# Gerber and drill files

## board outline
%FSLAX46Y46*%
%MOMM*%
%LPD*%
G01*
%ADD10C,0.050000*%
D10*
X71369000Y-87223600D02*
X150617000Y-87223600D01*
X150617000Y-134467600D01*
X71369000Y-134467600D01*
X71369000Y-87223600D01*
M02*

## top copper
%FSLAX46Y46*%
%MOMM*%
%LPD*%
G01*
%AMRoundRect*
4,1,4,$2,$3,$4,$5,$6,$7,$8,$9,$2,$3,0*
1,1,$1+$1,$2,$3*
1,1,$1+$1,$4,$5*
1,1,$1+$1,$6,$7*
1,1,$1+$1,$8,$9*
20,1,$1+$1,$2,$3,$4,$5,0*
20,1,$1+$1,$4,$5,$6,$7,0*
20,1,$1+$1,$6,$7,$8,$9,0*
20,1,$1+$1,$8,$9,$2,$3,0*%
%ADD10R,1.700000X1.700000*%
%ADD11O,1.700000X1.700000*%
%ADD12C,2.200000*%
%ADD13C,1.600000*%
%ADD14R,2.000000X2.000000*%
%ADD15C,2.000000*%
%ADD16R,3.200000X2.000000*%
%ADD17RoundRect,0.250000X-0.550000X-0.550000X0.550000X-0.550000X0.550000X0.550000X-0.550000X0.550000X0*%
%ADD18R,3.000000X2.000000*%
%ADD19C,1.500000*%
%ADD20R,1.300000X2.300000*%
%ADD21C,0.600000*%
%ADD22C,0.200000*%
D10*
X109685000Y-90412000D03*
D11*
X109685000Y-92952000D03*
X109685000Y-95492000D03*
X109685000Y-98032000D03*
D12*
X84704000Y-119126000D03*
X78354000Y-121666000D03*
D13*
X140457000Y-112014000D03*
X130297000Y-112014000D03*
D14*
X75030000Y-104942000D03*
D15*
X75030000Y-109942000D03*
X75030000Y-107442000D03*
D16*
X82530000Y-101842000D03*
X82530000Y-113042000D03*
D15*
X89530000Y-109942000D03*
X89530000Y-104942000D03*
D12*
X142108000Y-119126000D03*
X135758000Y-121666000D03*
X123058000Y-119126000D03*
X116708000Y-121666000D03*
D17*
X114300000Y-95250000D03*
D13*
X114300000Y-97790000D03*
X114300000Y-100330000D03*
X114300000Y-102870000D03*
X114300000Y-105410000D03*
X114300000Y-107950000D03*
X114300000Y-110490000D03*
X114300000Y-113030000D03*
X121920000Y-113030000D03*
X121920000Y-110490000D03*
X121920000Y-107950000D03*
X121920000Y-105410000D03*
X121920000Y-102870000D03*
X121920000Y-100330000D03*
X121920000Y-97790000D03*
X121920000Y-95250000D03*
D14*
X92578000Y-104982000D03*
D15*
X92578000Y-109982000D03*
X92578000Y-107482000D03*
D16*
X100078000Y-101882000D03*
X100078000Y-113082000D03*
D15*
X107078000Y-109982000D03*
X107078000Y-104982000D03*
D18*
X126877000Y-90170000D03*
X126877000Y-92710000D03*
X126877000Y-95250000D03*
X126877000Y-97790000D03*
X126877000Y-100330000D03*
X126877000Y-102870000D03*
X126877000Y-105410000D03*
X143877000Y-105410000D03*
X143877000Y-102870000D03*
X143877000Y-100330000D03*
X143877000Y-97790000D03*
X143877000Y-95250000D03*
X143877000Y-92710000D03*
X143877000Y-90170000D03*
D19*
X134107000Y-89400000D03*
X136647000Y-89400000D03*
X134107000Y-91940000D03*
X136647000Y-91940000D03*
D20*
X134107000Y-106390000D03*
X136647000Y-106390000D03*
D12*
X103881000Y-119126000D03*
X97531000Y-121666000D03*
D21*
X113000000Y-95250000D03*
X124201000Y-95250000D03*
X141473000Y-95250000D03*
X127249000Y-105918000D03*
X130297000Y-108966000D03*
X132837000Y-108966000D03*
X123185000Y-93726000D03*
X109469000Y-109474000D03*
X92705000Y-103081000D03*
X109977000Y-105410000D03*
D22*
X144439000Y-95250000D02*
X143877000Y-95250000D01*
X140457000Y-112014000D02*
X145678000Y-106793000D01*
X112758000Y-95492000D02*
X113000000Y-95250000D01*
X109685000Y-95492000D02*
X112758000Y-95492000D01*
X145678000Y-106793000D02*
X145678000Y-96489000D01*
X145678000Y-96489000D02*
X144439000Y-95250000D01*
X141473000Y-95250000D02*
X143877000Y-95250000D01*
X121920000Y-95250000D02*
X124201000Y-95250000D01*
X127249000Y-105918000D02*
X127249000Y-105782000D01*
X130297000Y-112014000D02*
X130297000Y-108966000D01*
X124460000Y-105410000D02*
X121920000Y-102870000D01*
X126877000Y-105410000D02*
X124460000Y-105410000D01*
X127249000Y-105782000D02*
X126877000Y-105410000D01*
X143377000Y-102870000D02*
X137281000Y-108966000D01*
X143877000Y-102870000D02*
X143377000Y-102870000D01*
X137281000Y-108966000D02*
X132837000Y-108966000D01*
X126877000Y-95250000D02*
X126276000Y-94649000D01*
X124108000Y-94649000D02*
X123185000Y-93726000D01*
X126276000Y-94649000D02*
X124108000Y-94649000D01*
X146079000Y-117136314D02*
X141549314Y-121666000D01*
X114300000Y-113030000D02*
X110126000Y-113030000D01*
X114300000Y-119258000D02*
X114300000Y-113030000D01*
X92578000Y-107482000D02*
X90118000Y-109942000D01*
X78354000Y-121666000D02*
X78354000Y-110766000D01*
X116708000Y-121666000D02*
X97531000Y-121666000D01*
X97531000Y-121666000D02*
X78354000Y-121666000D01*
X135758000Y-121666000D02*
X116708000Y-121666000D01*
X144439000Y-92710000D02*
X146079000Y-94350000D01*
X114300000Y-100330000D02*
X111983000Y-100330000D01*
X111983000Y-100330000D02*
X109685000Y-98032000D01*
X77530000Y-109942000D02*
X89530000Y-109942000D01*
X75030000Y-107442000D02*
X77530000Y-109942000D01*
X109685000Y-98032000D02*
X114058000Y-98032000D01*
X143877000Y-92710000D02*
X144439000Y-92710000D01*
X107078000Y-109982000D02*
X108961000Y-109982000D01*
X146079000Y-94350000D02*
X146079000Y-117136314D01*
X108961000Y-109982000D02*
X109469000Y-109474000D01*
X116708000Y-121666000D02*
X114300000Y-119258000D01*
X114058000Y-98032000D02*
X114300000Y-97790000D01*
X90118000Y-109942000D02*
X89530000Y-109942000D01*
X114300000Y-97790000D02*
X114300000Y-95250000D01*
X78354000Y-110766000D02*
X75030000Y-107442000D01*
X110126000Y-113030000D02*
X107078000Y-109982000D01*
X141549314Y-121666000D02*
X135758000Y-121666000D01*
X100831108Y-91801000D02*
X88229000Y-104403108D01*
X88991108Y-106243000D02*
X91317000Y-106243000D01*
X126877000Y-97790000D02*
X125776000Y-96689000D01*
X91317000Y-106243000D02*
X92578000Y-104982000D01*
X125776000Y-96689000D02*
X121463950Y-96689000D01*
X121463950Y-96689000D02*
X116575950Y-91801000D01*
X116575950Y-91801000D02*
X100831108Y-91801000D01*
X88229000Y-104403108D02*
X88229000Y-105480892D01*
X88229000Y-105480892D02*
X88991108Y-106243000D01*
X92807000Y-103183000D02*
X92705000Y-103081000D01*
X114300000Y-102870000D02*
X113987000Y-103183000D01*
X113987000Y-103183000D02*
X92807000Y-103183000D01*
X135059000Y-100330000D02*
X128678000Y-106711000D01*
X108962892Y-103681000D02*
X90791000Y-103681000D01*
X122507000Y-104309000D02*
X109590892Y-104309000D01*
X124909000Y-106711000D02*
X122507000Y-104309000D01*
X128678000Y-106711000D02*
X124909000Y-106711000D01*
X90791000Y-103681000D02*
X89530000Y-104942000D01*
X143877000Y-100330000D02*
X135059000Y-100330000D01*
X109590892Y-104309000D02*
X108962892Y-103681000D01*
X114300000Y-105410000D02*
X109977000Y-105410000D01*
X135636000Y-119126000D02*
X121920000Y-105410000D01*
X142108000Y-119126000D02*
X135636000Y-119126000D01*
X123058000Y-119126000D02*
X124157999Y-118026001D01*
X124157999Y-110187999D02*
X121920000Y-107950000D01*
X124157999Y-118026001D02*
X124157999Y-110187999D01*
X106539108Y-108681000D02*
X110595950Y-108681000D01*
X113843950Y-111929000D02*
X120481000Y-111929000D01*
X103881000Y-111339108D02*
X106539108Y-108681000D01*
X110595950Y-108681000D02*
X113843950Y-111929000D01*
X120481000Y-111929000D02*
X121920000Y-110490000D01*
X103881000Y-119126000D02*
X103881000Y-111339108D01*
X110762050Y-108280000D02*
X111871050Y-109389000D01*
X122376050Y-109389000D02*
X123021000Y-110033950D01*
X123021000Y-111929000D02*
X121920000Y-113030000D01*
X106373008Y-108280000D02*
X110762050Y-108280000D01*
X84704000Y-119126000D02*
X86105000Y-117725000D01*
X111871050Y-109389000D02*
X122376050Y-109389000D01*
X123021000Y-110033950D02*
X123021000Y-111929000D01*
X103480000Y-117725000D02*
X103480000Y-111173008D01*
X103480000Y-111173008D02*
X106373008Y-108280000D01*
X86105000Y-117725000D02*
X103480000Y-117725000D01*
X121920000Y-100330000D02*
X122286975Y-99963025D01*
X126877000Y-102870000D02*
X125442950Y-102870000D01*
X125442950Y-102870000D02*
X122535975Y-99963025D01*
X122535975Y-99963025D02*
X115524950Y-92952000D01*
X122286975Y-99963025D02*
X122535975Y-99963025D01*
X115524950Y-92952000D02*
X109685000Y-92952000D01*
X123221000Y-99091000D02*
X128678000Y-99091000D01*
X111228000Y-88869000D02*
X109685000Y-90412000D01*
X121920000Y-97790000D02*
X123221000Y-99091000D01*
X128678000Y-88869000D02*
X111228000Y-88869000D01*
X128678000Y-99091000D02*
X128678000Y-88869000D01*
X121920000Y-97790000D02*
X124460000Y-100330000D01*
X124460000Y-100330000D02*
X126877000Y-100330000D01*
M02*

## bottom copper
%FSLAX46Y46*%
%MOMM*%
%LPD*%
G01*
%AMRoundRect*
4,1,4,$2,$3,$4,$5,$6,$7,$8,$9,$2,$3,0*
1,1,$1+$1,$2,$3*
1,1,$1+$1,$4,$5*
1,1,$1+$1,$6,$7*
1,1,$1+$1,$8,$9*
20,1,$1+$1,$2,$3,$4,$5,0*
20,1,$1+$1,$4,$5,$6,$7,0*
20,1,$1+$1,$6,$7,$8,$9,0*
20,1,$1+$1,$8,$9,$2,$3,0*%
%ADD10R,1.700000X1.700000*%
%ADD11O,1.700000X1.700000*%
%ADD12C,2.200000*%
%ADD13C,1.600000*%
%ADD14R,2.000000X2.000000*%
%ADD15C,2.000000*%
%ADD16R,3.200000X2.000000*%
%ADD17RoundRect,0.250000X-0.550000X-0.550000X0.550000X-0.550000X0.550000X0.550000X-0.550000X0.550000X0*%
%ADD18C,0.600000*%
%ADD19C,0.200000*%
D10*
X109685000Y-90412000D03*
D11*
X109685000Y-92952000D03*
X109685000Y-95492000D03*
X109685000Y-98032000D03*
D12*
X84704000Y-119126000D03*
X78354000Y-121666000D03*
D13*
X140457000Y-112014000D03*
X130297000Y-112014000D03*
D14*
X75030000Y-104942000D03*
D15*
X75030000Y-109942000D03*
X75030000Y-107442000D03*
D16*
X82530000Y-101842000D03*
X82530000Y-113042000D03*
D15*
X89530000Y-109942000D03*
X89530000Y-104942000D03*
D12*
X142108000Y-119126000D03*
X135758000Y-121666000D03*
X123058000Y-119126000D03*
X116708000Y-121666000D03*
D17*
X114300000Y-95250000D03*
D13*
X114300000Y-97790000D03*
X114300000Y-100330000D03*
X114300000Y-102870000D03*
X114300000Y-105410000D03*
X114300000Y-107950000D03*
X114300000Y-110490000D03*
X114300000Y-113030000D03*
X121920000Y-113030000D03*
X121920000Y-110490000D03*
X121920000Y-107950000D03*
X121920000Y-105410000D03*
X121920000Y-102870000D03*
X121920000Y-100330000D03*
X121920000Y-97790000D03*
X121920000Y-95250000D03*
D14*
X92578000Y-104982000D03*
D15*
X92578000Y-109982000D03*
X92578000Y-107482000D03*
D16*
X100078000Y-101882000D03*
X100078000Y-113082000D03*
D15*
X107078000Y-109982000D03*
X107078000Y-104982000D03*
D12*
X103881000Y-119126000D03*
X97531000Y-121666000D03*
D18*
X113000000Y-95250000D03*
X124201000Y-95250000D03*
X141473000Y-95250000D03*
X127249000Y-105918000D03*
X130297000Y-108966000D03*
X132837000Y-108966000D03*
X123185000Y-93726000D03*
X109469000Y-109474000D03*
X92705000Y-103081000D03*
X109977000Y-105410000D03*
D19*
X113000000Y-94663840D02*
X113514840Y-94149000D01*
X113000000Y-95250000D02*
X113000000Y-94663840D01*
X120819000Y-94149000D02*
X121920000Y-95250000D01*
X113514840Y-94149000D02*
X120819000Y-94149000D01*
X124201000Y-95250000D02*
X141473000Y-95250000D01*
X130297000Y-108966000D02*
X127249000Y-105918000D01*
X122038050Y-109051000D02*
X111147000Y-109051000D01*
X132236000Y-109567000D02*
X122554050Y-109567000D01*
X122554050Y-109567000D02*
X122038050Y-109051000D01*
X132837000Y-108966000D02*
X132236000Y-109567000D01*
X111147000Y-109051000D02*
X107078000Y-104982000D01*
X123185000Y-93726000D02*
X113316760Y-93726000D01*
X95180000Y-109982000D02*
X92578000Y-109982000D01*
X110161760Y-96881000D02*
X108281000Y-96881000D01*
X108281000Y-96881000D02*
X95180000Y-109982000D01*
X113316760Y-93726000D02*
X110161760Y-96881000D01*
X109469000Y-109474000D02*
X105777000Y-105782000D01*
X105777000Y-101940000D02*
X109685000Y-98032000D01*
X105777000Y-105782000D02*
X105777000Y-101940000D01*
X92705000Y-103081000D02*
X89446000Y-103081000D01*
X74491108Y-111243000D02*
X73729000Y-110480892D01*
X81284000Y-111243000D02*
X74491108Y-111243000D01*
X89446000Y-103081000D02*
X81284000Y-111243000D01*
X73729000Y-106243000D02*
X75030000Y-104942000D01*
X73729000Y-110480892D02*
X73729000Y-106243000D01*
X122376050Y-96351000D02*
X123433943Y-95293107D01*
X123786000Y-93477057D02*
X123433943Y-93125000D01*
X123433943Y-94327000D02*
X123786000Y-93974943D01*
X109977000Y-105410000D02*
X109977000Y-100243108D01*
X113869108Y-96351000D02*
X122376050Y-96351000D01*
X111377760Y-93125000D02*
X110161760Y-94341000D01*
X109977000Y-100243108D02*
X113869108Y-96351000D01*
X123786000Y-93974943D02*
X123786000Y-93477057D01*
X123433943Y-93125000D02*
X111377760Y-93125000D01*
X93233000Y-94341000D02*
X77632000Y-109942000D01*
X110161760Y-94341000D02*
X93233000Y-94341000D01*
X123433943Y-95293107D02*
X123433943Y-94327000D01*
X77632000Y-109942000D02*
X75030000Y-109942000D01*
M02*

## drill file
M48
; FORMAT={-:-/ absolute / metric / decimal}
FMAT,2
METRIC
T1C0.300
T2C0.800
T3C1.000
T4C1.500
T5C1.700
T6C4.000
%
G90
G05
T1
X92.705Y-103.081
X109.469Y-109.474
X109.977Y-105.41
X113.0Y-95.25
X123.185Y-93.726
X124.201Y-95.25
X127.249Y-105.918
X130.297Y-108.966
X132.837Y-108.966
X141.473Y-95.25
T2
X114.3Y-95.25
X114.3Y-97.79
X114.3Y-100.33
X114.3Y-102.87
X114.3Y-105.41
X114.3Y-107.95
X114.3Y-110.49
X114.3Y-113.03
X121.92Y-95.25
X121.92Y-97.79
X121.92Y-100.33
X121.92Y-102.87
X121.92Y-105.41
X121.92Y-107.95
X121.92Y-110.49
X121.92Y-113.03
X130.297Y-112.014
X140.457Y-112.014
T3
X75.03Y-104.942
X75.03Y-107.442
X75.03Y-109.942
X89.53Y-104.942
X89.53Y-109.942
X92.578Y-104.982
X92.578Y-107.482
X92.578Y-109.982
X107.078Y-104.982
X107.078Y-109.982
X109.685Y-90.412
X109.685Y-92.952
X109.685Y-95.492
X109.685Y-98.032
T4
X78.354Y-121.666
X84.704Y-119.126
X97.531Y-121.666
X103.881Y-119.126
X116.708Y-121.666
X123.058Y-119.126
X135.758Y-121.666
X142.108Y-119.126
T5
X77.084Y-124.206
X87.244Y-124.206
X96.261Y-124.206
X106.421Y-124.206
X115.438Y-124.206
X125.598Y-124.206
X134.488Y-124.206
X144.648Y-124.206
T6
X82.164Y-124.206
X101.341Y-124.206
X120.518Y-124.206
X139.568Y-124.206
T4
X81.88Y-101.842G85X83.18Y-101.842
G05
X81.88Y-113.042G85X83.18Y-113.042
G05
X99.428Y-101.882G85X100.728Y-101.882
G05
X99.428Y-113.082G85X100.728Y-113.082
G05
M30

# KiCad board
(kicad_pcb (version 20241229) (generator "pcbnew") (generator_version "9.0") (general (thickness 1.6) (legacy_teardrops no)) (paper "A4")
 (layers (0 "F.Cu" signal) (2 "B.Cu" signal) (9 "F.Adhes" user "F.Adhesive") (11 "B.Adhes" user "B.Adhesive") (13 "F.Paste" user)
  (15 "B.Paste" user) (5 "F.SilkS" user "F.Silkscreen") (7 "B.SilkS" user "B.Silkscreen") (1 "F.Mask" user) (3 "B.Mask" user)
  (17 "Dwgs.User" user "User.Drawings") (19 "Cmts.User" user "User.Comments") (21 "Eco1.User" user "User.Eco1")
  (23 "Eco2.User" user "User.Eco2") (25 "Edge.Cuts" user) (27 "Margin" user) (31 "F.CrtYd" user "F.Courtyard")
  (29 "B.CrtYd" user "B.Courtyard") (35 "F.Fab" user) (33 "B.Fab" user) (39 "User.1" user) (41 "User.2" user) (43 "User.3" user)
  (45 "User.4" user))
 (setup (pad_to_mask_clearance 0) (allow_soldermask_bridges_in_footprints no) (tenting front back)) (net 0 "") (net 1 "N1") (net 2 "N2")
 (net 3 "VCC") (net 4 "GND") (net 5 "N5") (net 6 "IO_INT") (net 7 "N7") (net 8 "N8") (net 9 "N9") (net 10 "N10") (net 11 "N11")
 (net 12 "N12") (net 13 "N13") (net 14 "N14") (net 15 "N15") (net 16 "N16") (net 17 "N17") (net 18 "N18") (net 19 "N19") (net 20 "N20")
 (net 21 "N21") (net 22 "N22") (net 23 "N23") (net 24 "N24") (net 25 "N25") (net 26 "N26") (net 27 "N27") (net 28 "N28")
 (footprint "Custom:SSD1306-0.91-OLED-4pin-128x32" (layer "F.Cu") (at 73.185 88.222)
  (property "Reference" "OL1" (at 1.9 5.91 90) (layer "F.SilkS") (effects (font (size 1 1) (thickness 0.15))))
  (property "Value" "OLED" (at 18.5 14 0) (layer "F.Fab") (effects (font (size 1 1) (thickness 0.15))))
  (pad "1" thru_hole rect (at 36.5 2.19) (size 1.7 1.7) (drill 1) (layers "*.Cu" "*.Mask") (remove_unused_layers no) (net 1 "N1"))
  (pad "2" thru_hole oval (at 36.5 4.73) (size 1.7 1.7) (drill 1) (layers "*.Cu" "*.Mask") (remove_unused_layers no) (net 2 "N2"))
  (pad "3" thru_hole oval (at 36.5 7.27) (size 1.7 1.7) (drill 1) (layers "*.Cu" "*.Mask") (remove_unused_layers no) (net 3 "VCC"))
  (pad "4" thru_hole oval (at 36.5 9.81) (size 1.7 1.7) (drill 1) (layers "*.Cu" "*.Mask") (remove_unused_layers no) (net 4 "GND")))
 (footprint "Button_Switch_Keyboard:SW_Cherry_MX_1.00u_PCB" (layer "F.Cu") (at 84.704 119.126)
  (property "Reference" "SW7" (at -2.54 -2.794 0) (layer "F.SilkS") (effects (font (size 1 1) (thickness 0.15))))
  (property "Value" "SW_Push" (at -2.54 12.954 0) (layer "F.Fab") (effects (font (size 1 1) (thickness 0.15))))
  (pad "" np_thru_hole circle (at -7.62 5.08) (size 1.7 1.7) (drill 1.7) (layers "*.Cu" "*.Mask"))
  (pad "" np_thru_hole circle (at -2.54 5.08) (size 4 4) (drill 4) (layers "*.Cu" "*.Mask"))
  (pad "" np_thru_hole circle (at 2.54 5.08) (size 1.7 1.7) (drill 1.7) (layers "*.Cu" "*.Mask"))
  (pad "1" thru_hole circle (at 0 0) (size 2.2 2.2) (drill 1.5) (layers "*.Cu" "*.Mask") (remove_unused_layers no) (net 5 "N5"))
  (pad "2" thru_hole circle (at -6.35 2.54) (size 2.2 2.2) (drill 1.5) (layers "*.Cu" "*.Mask") (remove_unused_layers no) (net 4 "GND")))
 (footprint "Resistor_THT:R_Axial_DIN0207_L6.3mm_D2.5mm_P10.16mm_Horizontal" (layer "F.Cu") (at 140.457 112.014 180)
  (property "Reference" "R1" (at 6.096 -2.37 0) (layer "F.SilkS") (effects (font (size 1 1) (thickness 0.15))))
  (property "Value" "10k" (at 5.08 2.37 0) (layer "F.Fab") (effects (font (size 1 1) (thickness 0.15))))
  (pad "1" thru_hole circle (at 0 0 180) (size 1.6 1.6) (drill 0.8) (layers "*.Cu" "*.Mask") (remove_unused_layers no) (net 3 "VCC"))
  (pad "2" thru_hole circle (at 10.16 0 180) (size 1.6 1.6) (drill 0.8) (layers "*.Cu" "*.Mask") (remove_unused_layers no) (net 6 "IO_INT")))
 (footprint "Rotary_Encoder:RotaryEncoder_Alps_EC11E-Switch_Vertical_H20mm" (layer "F.Cu") (at 75.03 104.942)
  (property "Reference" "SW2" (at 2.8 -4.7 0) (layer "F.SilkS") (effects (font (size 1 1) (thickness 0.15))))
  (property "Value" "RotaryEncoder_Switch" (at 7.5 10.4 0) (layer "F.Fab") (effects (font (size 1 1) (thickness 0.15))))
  (pad "A" thru_hole rect (at 0 0) (size 2 2) (drill 1) (layers "*.Cu" "*.Mask") (remove_unused_layers no) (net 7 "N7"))
  (pad "B" thru_hole circle (at 0 5) (size 2 2) (drill 1) (layers "*.Cu" "*.Mask") (remove_unused_layers no) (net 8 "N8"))
  (pad "C" thru_hole circle (at 0 2.5) (size 2 2) (drill 1) (layers "*.Cu" "*.Mask") (remove_unused_layers no) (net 4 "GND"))
  (pad "MP" thru_hole rect (at 7.5 -3.1) (size 3.2 2) (drill oval 2.8 1.5) (layers "*.Cu" "*.Mask") (remove_unused_layers no))
  (pad "MP" thru_hole rect (at 7.5 8.1) (size 3.2 2) (drill oval 2.8 1.5) (layers "*.Cu" "*.Mask") (remove_unused_layers no))
  (pad "S1" thru_hole circle (at 14.5 5) (size 2 2) (drill 1) (layers "*.Cu" "*.Mask") (remove_unused_layers no) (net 4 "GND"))
  (pad "S2" thru_hole circle (at 14.5 0) (size 2 2) (drill 1) (layers "*.Cu" "*.Mask") (remove_unused_layers no) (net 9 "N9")))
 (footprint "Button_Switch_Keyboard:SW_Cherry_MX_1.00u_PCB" (layer "F.Cu") (at 142.108 119.126)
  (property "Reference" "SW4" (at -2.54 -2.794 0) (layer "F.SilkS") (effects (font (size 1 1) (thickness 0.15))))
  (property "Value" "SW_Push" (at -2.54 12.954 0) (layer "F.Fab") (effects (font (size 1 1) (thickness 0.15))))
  (pad "" np_thru_hole circle (at -7.62 5.08) (size 1.7 1.7) (drill 1.7) (layers "*.Cu" "*.Mask"))
  (pad "" np_thru_hole circle (at -2.54 5.08) (size 4 4) (drill 4) (layers "*.Cu" "*.Mask"))
  (pad "" np_thru_hole circle (at 2.54 5.08) (size 1.7 1.7) (drill 1.7) (layers "*.Cu" "*.Mask"))
  (pad "1" thru_hole circle (at 0 0) (size 2.2 2.2) (drill 1.5) (layers "*.Cu" "*.Mask") (remove_unused_layers no) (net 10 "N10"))
  (pad "2" thru_hole circle (at -6.35 2.54) (size 2.2 2.2) (drill 1.5) (layers "*.Cu" "*.Mask") (remove_unused_layers no) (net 4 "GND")))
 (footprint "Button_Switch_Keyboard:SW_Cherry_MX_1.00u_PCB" (layer "F.Cu") (at 123.058 119.126)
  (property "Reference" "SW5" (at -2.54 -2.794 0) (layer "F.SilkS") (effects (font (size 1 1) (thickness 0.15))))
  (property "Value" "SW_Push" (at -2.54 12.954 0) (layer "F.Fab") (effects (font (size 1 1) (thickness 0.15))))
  (pad "" np_thru_hole circle (at -7.62 5.08) (size 1.7 1.7) (drill 1.7) (layers "*.Cu" "*.Mask"))
  (pad "" np_thru_hole circle (at -2.54 5.08) (size 4 4) (drill 4) (layers "*.Cu" "*.Mask"))
  (pad "" np_thru_hole circle (at 2.54 5.08) (size 1.7 1.7) (drill 1.7) (layers "*.Cu" "*.Mask"))
  (pad "1" thru_hole circle (at 0 0) (size 2.2 2.2) (drill 1.5) (layers "*.Cu" "*.Mask") (remove_unused_layers no) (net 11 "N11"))
  (pad "2" thru_hole circle (at -6.35 2.54) (size 2.2 2.2) (drill 1.5) (layers "*.Cu" "*.Mask") (remove_unused_layers no) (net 4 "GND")))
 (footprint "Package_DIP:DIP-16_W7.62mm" (layer "F.Cu") (at 114.3 95.25)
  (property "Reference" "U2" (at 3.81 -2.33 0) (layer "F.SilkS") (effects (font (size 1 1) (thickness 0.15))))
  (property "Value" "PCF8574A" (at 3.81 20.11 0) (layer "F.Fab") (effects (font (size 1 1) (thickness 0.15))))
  (pad "1" thru_hole roundrect (at 0 0) (size 1.6 1.6) (drill 0.8) (layers "*.Cu" "*.Mask") (remove_unused_layers no)
   (roundrect_rratio 0.15625) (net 4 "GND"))
  (pad "2" thru_hole circle (at 0 2.54) (size 1.6 1.6) (drill 0.8) (layers "*.Cu" "*.Mask") (remove_unused_layers no) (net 4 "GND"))
  (pad "3" thru_hole circle (at 0 5.08) (size 1.6 1.6) (drill 0.8) (layers "*.Cu" "*.Mask") (remove_unused_layers no) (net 4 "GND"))
  (pad "4" thru_hole circle (at 0 7.62) (size 1.6 1.6) (drill 0.8) (layers "*.Cu" "*.Mask") (remove_unused_layers no) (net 7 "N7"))
  (pad "5" thru_hole circle (at 0 10.16) (size 1.6 1.6) (drill 0.8) (layers "*.Cu" "*.Mask") (remove_unused_layers no) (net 8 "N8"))
  (pad "6" thru_hole circle (at 0 12.7) (size 1.6 1.6) (drill 0.8) (layers "*.Cu" "*.Mask") (remove_unused_layers no) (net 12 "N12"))
  (pad "7" thru_hole circle (at 0 15.24) (size 1.6 1.6) (drill 0.8) (layers "*.Cu" "*.Mask") (remove_unused_layers no) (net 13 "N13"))
  (pad "8" thru_hole circle (at 0 17.78) (size 1.6 1.6) (drill 0.8) (layers "*.Cu" "*.Mask") (remove_unused_layers no) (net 4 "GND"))
  (pad "9" thru_hole circle (at 7.62 17.78) (size 1.6 1.6) (drill 0.8) (layers "*.Cu" "*.Mask") (remove_unused_layers no) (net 5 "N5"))
  (pad "10" thru_hole circle (at 7.62 15.24) (size 1.6 1.6) (drill 0.8) (layers "*.Cu" "*.Mask") (remove_unused_layers no) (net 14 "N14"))
  (pad "11" thru_hole circle (at 7.62 12.7) (size 1.6 1.6) (drill 0.8) (layers "*.Cu" "*.Mask") (remove_unused_layers no) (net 11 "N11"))
  (pad "12" thru_hole circle (at 7.62 10.16) (size 1.6 1.6) (drill 0.8) (layers "*.Cu" "*.Mask") (remove_unused_layers no) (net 10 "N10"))
  (pad "13" thru_hole circle (at 7.62 7.62) (size 1.6 1.6) (drill 0.8) (layers "*.Cu" "*.Mask") (remove_unused_layers no) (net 6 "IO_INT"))
  (pad "14" thru_hole circle (at 7.62 5.08) (size 1.6 1.6) (drill 0.8) (layers "*.Cu" "*.Mask") (remove_unused_layers no) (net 2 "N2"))
  (pad "15" thru_hole circle (at 7.62 2.54) (size 1.6 1.6) (drill 0.8) (layers "*.Cu" "*.Mask") (remove_unused_layers no) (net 1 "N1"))
  (pad "16" thru_hole circle (at 7.62 0) (size 1.6 1.6) (drill 0.8) (layers "*.Cu" "*.Mask") (remove_unused_layers no) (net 3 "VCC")))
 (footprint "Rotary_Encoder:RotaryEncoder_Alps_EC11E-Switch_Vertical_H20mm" (layer "F.Cu") (at 92.578 104.982)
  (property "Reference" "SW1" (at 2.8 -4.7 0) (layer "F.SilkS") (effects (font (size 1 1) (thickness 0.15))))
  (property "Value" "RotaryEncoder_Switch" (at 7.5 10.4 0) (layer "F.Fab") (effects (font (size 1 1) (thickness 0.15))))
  (pad "A" thru_hole rect (at 0 0) (size 2 2) (drill 1) (layers "*.Cu" "*.Mask") (remove_unused_layers no) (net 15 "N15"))
  (pad "B" thru_hole circle (at 0 5) (size 2 2) (drill 1) (layers "*.Cu" "*.Mask") (remove_unused_layers no) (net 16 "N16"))
  (pad "C" thru_hole circle (at 0 2.5) (size 2 2) (drill 1) (layers "*.Cu" "*.Mask") (remove_unused_layers no) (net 4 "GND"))
  (pad "MP" thru_hole rect (at 7.5 -3.1) (size 3.2 2) (drill oval 2.8 1.5) (layers "*.Cu" "*.Mask") (remove_unused_layers no))
  (pad "MP" thru_hole rect (at 7.5 8.1) (size 3.2 2) (drill oval 2.8 1.5) (layers "*.Cu" "*.Mask") (remove_unused_layers no))
  (pad "S1" thru_hole circle (at 14.5 5) (size 2 2) (drill 1) (layers "*.Cu" "*.Mask") (remove_unused_layers no) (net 4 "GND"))
  (pad "S2" thru_hole circle (at 14.5 0) (size 2 2) (drill 1) (layers "*.Cu" "*.Mask") (remove_unused_layers no) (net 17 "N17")))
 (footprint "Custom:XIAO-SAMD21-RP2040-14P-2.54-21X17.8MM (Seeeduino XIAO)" (layer "F.Cu") (at 135.377 97.79)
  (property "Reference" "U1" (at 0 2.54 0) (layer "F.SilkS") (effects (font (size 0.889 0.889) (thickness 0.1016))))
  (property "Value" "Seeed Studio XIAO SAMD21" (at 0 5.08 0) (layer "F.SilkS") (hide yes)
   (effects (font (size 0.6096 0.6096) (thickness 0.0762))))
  (pad "1" smd rect (at -8.5 -7.62) (size 3 2) (layers "F.Cu" "F.Mask" "F.Paste") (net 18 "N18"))
  (pad "2" smd rect (at -8.5 -5.08) (size 3 2) (layers "F.Cu" "F.Mask" "F.Paste") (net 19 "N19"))
  (pad "3" smd rect (at -8.5 -2.54) (size 3 2) (layers "F.Cu" "F.Mask" "F.Paste") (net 16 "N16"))
  (pad "4" smd rect (at -8.5 0) (size 3 2) (layers "F.Cu" "F.Mask" "F.Paste") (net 15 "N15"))
  (pad "5" smd rect (at -8.5 2.54) (size 3 2) (layers "F.Cu" "F.Mask" "F.Paste") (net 1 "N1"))
  (pad "6" smd rect (at -8.5 5.08 180) (size 3 2) (layers "F.Cu" "F.Mask" "F.Paste") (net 2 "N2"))
  (pad "7" smd rect (at -8.5 7.62) (size 3 2) (layers "F.Cu" "F.Mask" "F.Paste") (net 6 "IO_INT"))
  (pad "8" smd rect (at 8.5 7.62) (size 3 2) (layers "F.Cu" "F.Mask" "F.Paste") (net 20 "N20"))
  (pad "9" smd rect (at 8.5 5.08) (size 3 2) (layers "F.Cu" "F.Mask" "F.Paste") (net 17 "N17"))
  (pad "10" smd rect (at 8.5 2.54) (size 3 2) (layers "F.Cu" "F.Mask" "F.Paste") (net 9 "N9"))
  (pad "11" smd rect (at 8.5 0) (size 3 2) (layers "F.Cu" "F.Mask" "F.Paste") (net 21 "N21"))
  (pad "12" smd rect (at 8.5 -2.54) (size 3 2) (layers "F.Cu" "F.Mask" "F.Paste") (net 3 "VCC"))
  (pad "13" smd rect (at 8.5 -5.08) (size 3 2) (layers "F.Cu" "F.Mask" "F.Paste") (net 4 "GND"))
  (pad "14" smd rect (at 8.5 -7.62) (size 3 2) (layers "F.Cu" "F.Mask" "F.Paste") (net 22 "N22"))
  (pad "15" smd circle (at -1.27 -8.39 90) (size 1.5 1.5) (layers "F.Cu" "F.Mask" "F.Paste") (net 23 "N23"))
  (pad "16" smd circle (at 1.27 -8.39 90) (size 1.5 1.5) (layers "F.Cu" "F.Mask" "F.Paste") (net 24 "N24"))
  (pad "17" smd circle (at -1.27 -5.85 90) (size 1.5 1.5) (layers "F.Cu" "F.Mask" "F.Paste") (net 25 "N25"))
  (pad "18" smd circle (at 1.27 -5.85 90) (size 1.5 1.5) (layers "F.Cu" "F.Mask" "F.Paste") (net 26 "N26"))
  (pad "19" smd rect (at -1.27 8.6 90) (size 2.3 1.3) (layers "F.Cu" "F.Mask" "F.Paste") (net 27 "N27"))
  (pad "20" smd rect (at 1.27 8.6 90) (size 2.3 1.3) (layers "F.Cu" "F.Mask" "F.Paste") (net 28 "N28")))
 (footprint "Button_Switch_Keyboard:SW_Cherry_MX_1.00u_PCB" (layer "F.Cu") (at 103.881 119.126)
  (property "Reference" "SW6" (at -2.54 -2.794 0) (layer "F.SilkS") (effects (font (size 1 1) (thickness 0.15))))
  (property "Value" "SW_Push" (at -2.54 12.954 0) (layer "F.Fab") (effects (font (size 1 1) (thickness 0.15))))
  (pad "" np_thru_hole circle (at -7.62 5.08) (size 1.7 1.7) (drill 1.7) (layers "*.Cu" "*.Mask"))
  (pad "" np_thru_hole circle (at -2.54 5.08) (size 4 4) (drill 4) (layers "*.Cu" "*.Mask"))
  (pad "" np_thru_hole circle (at 2.54 5.08) (size 1.7 1.7) (drill 1.7) (layers "*.Cu" "*.Mask"))
  (pad "1" thru_hole circle (at 0 0) (size 2.2 2.2) (drill 1.5) (layers "*.Cu" "*.Mask") (remove_unused_layers no) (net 14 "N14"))
  (pad "2" thru_hole circle (at -6.35 2.54) (size 2.2 2.2) (drill 1.5) (layers "*.Cu" "*.Mask") (remove_unused_layers no) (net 4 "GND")))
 (gr_rect (start 71.369 87.2236) (end 150.617 134.4676) (stroke (width 0.05) (type default)) (fill no) (layer "Edge.Cuts"))
 (segment (start 144.439 95.25) (end 143.877 95.25) (width 0.2) (layer "F.Cu") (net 3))
 (segment (start 140.457 112.014) (end 145.678 106.793) (width 0.2) (layer "F.Cu") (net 3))
 (segment (start 112.758 95.492) (end 113 95.25) (width 0.2) (layer "F.Cu") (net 3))
 (segment (start 109.685 95.492) (end 112.758 95.492) (width 0.2) (layer "F.Cu") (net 3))
 (segment (start 145.678 106.793) (end 145.678 96.489) (width 0.2) (layer "F.Cu") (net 3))
 (segment (start 145.678 96.489) (end 144.439 95.25) (width 0.2) (layer "F.Cu") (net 3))
 (segment (start 141.473 95.25) (end 143.877 95.25) (width 0.2) (layer "F.Cu") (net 3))
 (segment (start 121.92 95.25) (end 124.201 95.25) (width 0.2) (layer "F.Cu") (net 3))
 (via (at 113 95.25) (size 0.6) (drill 0.3) (layers "F.Cu" "B.Cu") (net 3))
 (via (at 124.201 95.25) (size 0.6) (drill 0.3) (layers "F.Cu" "B.Cu") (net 3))
 (via (at 141.473 95.25) (size 0.6) (drill 0.3) (layers "F.Cu" "B.Cu") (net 3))
 (segment (start 113 94.66384) (end 113.51484 94.149) (width 0.2) (layer "B.Cu") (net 3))
 (segment (start 113 95.25) (end 113 94.66384) (width 0.2) (layer "B.Cu") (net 3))
 (segment (start 120.819 94.149) (end 121.92 95.25) (width 0.2) (layer "B.Cu") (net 3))
 (segment (start 113.51484 94.149) (end 120.819 94.149) (width 0.2) (layer "B.Cu") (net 3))
 (segment (start 124.201 95.25) (end 141.473 95.25) (width 0.2) (layer "B.Cu") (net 3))
 (segment (start 127.249 105.918) (end 127.249 105.782) (width 0.2) (layer "F.Cu") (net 6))
 (segment (start 130.297 112.014) (end 130.297 108.966) (width 0.2) (layer "F.Cu") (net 6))
 (segment (start 124.46 105.41) (end 121.92 102.87) (width 0.2) (layer "F.Cu") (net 6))
 (segment (start 126.877 105.41) (end 124.46 105.41) (width 0.2) (layer "F.Cu") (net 6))
 (segment (start 127.249 105.782) (end 126.877 105.41) (width 0.2) (layer "F.Cu") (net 6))
 (via (at 127.249 105.918) (size 0.6) (drill 0.3) (layers "F.Cu" "B.Cu") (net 6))
 (via (at 130.297 108.966) (size 0.6) (drill 0.3) (layers "F.Cu" "B.Cu") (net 6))
 (segment (start 130.297 108.966) (end 127.249 105.918) (width 0.2) (layer "B.Cu") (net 6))
 (segment (start 143.377 102.87) (end 137.281 108.966) (width 0.2) (layer "F.Cu") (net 17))
 (segment (start 143.877 102.87) (end 143.377 102.87) (width 0.2) (layer "F.Cu") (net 17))
 (segment (start 137.281 108.966) (end 132.837 108.966) (width 0.2) (layer "F.Cu") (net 17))
 (via (at 132.837 108.966) (size 0.6) (drill 0.3) (layers "F.Cu" "B.Cu") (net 17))
 (segment (start 122.03805 109.051) (end 111.147 109.051) (width 0.2) (layer "B.Cu") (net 17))
 (segment (start 132.236 109.567) (end 122.55405 109.567) (width 0.2) (layer "B.Cu") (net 17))
 (segment (start 122.55405 109.567) (end 122.03805 109.051) (width 0.2) (layer "B.Cu") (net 17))
 (segment (start 132.837 108.966) (end 132.236 109.567) (width 0.2) (layer "B.Cu") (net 17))
 (segment (start 111.147 109.051) (end 107.078 104.982) (width 0.2) (layer "B.Cu") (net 17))
 (segment (start 126.877 95.25) (end 126.276 94.649) (width 0.2) (layer "F.Cu") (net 16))
 (segment (start 124.108 94.649) (end 123.185 93.726) (width 0.2) (layer "F.Cu") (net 16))
 (segment (start 126.276 94.649) (end 124.108 94.649) (width 0.2) (layer "F.Cu") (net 16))
 (via (at 123.185 93.726) (size 0.6) (drill 0.3) (layers "F.Cu" "B.Cu") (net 16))
 (segment (start 123.185 93.726) (end 113.31676 93.726) (width 0.2) (layer "B.Cu") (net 16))
 (segment (start 95.18 109.982) (end 92.578 109.982) (width 0.2) (layer "B.Cu") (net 16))
 (segment (start 110.16176 96.881) (end 108.281 96.881) (width 0.2) (layer "B.Cu") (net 16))
 (segment (start 108.281 96.881) (end 95.18 109.982) (width 0.2) (layer "B.Cu") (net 16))
 (segment (start 113.31676 93.726) (end 110.16176 96.881) (width 0.2) (layer "B.Cu") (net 16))
 (segment (start 146.079 117.136314) (end 141.549314 121.666) (width 0.2) (layer "F.Cu") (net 4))
 (segment (start 114.3 113.03) (end 110.126 113.03) (width 0.2) (layer "F.Cu") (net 4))
 (segment (start 114.3 119.258) (end 114.3 113.03) (width 0.2) (layer "F.Cu") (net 4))
 (segment (start 92.578 107.482) (end 90.118 109.942) (width 0.2) (layer "F.Cu") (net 4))
 (segment (start 78.354 121.666) (end 78.354 110.766) (width 0.2) (layer "F.Cu") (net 4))
 (segment (start 116.708 121.666) (end 97.531 121.666) (width 0.2) (layer "F.Cu") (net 4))
 (segment (start 97.531 121.666) (end 78.354 121.666) (width 0.2) (layer "F.Cu") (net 4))
 (segment (start 135.758 121.666) (end 116.708 121.666) (width 0.2) (layer "F.Cu") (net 4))
 (segment (start 144.439 92.71) (end 146.079 94.35) (width 0.2) (layer "F.Cu") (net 4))
 (segment (start 114.3 100.33) (end 111.983 100.33) (width 0.2) (layer "F.Cu") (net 4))
 (segment (start 111.983 100.33) (end 109.685 98.032) (width 0.2) (layer "F.Cu") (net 4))
 (segment (start 77.53 109.942) (end 89.53 109.942) (width 0.2) (layer "F.Cu") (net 4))
 (segment (start 75.03 107.442) (end 77.53 109.942) (width 0.2) (layer "F.Cu") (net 4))
 (segment (start 109.685 98.032) (end 114.058 98.032) (width 0.2) (layer "F.Cu") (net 4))
 (segment (start 143.877 92.71) (end 144.439 92.71) (width 0.2) (layer "F.Cu") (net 4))
 (segment (start 107.078 109.982) (end 108.961 109.982) (width 0.2) (layer "F.Cu") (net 4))
 (segment (start 146.079 94.35) (end 146.079 117.136314) (width 0.2) (layer "F.Cu") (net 4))
 (segment (start 108.961 109.982) (end 109.469 109.474) (width 0.2) (layer "F.Cu") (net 4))
 (segment (start 116.708 121.666) (end 114.3 119.258) (width 0.2) (layer "F.Cu") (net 4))
 (segment (start 114.058 98.032) (end 114.3 97.79) (width 0.2) (layer "F.Cu") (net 4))
 (segment (start 90.118 109.942) (end 89.53 109.942) (width 0.2) (layer "F.Cu") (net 4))
 (segment (start 114.3 97.79) (end 114.3 95.25) (width 0.2) (layer "F.Cu") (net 4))
 (segment (start 78.354 110.766) (end 75.03 107.442) (width 0.2) (layer "F.Cu") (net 4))
 (segment (start 110.126 113.03) (end 107.078 109.982) (width 0.2) (layer "F.Cu") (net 4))
 (segment (start 141.549314 121.666) (end 135.758 121.666) (width 0.2) (layer "F.Cu") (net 4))
 (via (at 109.469 109.474) (size 0.6) (drill 0.3) (layers "F.Cu" "B.Cu") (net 4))
 (segment (start 109.469 109.474) (end 105.777 105.782) (width 0.2) (layer "B.Cu") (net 4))
 (segment (start 105.777 101.94) (end 109.685 98.032) (width 0.2) (layer "B.Cu") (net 4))
 (segment (start 105.777 105.782) (end 105.777 101.94) (width 0.2) (layer "B.Cu") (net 4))
 (segment (start 100.831108 91.801) (end 88.229 104.403108) (width 0.2) (layer "F.Cu") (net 15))
 (segment (start 88.991108 106.243) (end 91.317 106.243) (width 0.2) (layer "F.Cu") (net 15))
 (segment (start 126.877 97.79) (end 125.776 96.689) (width 0.2) (layer "F.Cu") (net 15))
 (segment (start 91.317 106.243) (end 92.578 104.982) (width 0.2) (layer "F.Cu") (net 15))
 (segment (start 125.776 96.689) (end 121.46395 96.689) (width 0.2) (layer "F.Cu") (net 15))
 (segment (start 121.46395 96.689) (end 116.57595 91.801) (width 0.2) (layer "F.Cu") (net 15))
 (segment (start 116.57595 91.801) (end 100.831108 91.801) (width 0.2) (layer "F.Cu") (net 15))
 (segment (start 88.229 104.403108) (end 88.229 105.480892) (width 0.2) (layer "F.Cu") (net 15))
 (segment (start 88.229 105.480892) (end 88.991108 106.243) (width 0.2) (layer "F.Cu") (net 15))
 (segment (start 92.807 103.183) (end 92.705 103.081) (width 0.2) (layer "F.Cu") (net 7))
 (segment (start 114.3 102.87) (end 113.987 103.183) (width 0.2) (layer "F.Cu") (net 7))
 (segment (start 113.987 103.183) (end 92.807 103.183) (width 0.2) (layer "F.Cu") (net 7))
 (via (at 92.705 103.081) (size 0.6) (drill 0.3) (layers "F.Cu" "B.Cu") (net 7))
 (segment (start 92.705 103.081) (end 89.446 103.081) (width 0.2) (layer "B.Cu") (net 7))
 (segment (start 74.491108 111.243) (end 73.729 110.480892) (width 0.2) (layer "B.Cu") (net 7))
 (segment (start 81.284 111.243) (end 74.491108 111.243) (width 0.2) (layer "B.Cu") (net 7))
 (segment (start 89.446 103.081) (end 81.284 111.243) (width 0.2) (layer "B.Cu") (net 7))
 (segment (start 73.729 106.243) (end 75.03 104.942) (width 0.2) (layer "B.Cu") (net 7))
 (segment (start 73.729 110.480892) (end 73.729 106.243) (width 0.2) (layer "B.Cu") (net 7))
 (segment (start 135.059 100.33) (end 128.678 106.711) (width 0.2) (layer "F.Cu") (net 9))
 (segment (start 108.962892 103.681) (end 90.791 103.681) (width 0.2) (layer "F.Cu") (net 9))
 (segment (start 122.507 104.309) (end 109.590892 104.309) (width 0.2) (layer "F.Cu") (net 9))
 (segment (start 124.909 106.711) (end 122.507 104.309) (width 0.2) (layer "F.Cu") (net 9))
 (segment (start 128.678 106.711) (end 124.909 106.711) (width 0.2) (layer "F.Cu") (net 9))
 (segment (start 90.791 103.681) (end 89.53 104.942) (width 0.2) (layer "F.Cu") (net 9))
 (segment (start 143.877 100.33) (end 135.059 100.33) (width 0.2) (layer "F.Cu") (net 9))
 (segment (start 109.590892 104.309) (end 108.962892 103.681) (width 0.2) (layer "F.Cu") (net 9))
 (segment (start 114.3 105.41) (end 109.977 105.41) (width 0.2) (layer "F.Cu") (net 8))
 (via (at 109.977 105.41) (size 0.6) (drill 0.3) (layers "F.Cu" "B.Cu") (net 8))
 (segment (start 122.37605 96.351) (end 123.433943 95.293107) (width 0.2) (layer "B.Cu") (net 8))
 (segment (start 123.786 93.477057) (end 123.433943 93.125) (width 0.2) (layer "B.Cu") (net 8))
 (segment (start 123.433943 94.327) (end 123.786 93.974943) (width 0.2) (layer "B.Cu") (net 8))
 (segment (start 109.977 105.41) (end 109.977 100.243108) (width 0.2) (layer "B.Cu") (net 8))
 (segment (start 113.869108 96.351) (end 122.37605 96.351) (width 0.2) (layer "B.Cu") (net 8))
 (segment (start 111.37776 93.125) (end 110.16176 94.341) (width 0.2) (layer "B.Cu") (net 8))
 (segment (start 109.977 100.243108) (end 113.869108 96.351) (width 0.2) (layer "B.Cu") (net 8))
 (segment (start 123.786 93.974943) (end 123.786 93.477057) (width 0.2) (layer "B.Cu") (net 8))
 (segment (start 123.433943 93.125) (end 111.37776 93.125) (width 0.2) (layer "B.Cu") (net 8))
 (segment (start 93.233 94.341) (end 77.632 109.942) (width 0.2) (layer "B.Cu") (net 8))
 (segment (start 110.16176 94.341) (end 93.233 94.341) (width 0.2) (layer "B.Cu") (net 8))
 (segment (start 123.433943 95.293107) (end 123.433943 94.327) (width 0.2) (layer "B.Cu") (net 8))
 (segment (start 77.632 109.942) (end 75.03 109.942) (width 0.2) (layer "B.Cu") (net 8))
 (segment (start 135.636 119.126) (end 121.92 105.41) (width 0.2) (layer "F.Cu") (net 10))
 (segment (start 142.108 119.126) (end 135.636 119.126) (width 0.2) (layer "F.Cu") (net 10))
 (segment (start 123.058 119.126) (end 124.157999 118.026001) (width 0.2) (layer "F.Cu") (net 11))
 (segment (start 124.157999 110.187999) (end 121.92 107.95) (width 0.2) (layer "F.Cu") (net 11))
 (segment (start 124.157999 118.026001) (end 124.157999 110.187999) (width 0.2) (layer "F.Cu") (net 11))
 (segment (start 106.539108 108.681) (end 110.59595 108.681) (width 0.2) (layer "F.Cu") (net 14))
 (segment (start 113.84395 111.929) (end 120.481 111.929) (width 0.2) (layer "F.Cu") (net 14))
 (segment (start 103.881 111.339108) (end 106.539108 108.681) (width 0.2) (layer "F.Cu") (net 14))
 (segment (start 110.59595 108.681) (end 113.84395 111.929) (width 0.2) (layer "F.Cu") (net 14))
 (segment (start 120.481 111.929) (end 121.92 110.49) (width 0.2) (layer "F.Cu") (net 14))
 (segment (start 103.881 119.126) (end 103.881 111.339108) (width 0.2) (layer "F.Cu") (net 14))
 (segment (start 110.76205 108.28) (end 111.87105 109.389) (width 0.2) (layer "F.Cu") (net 5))
 (segment (start 122.37605 109.389) (end 123.021 110.03395) (width 0.2) (layer "F.Cu") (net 5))
 (segment (start 123.021 111.929) (end 121.92 113.03) (width 0.2) (layer "F.Cu") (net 5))
 (segment (start 106.373008 108.28) (end 110.76205 108.28) (width 0.2) (layer "F.Cu") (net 5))
 (segment (start 84.704 119.126) (end 86.105 117.725) (width 0.2) (layer "F.Cu") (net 5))
 (segment (start 111.87105 109.389) (end 122.37605 109.389) (width 0.2) (layer "F.Cu") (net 5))
 (segment (start 123.021 110.03395) (end 123.021 111.929) (width 0.2) (layer "F.Cu") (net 5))
 (segment (start 103.48 117.725) (end 103.48 111.173008) (width 0.2) (layer "F.Cu") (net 5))
 (segment (start 103.48 111.173008) (end 106.373008 108.28) (width 0.2) (layer "F.Cu") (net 5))
 (segment (start 86.105 117.725) (end 103.48 117.725) (width 0.2) (layer "F.Cu") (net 5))
 (segment (start 121.92 100.33) (end 122.286975 99.963025) (width 0.2) (layer "F.Cu") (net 2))
 (segment (start 126.877 102.87) (end 125.44295 102.87) (width 0.2) (layer "F.Cu") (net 2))
 (segment (start 125.44295 102.87) (end 122.535975 99.963025) (width 0.2) (layer "F.Cu") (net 2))
 (segment (start 122.535975 99.963025) (end 115.52495 92.952) (width 0.2) (layer "F.Cu") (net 2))
 (segment (start 122.286975 99.963025) (end 122.535975 99.963025) (width 0.2) (layer "F.Cu") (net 2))
 (segment (start 115.52495 92.952) (end 109.685 92.952) (width 0.2) (layer "F.Cu") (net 2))
 (segment (start 123.221 99.091) (end 128.678 99.091) (width 0.2) (layer "F.Cu") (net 1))
 (segment (start 111.228 88.869) (end 109.685 90.412) (width 0.2) (layer "F.Cu") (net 1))
 (segment (start 121.92 97.79) (end 123.221 99.091) (width 0.2) (layer "F.Cu") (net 1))
 (segment (start 128.678 88.869) (end 111.228 88.869) (width 0.2) (layer "F.Cu") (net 1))
 (segment (start 128.678 99.091) (end 128.678 88.869) (width 0.2) (layer "F.Cu") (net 1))
 (segment (start 121.92 97.79) (end 124.46 100.33) (width 0.2) (layer "F.Cu") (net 1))
 (segment (start 124.46 100.33) (end 126.877 100.33) (width 0.2) (layer "F.Cu") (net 1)))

